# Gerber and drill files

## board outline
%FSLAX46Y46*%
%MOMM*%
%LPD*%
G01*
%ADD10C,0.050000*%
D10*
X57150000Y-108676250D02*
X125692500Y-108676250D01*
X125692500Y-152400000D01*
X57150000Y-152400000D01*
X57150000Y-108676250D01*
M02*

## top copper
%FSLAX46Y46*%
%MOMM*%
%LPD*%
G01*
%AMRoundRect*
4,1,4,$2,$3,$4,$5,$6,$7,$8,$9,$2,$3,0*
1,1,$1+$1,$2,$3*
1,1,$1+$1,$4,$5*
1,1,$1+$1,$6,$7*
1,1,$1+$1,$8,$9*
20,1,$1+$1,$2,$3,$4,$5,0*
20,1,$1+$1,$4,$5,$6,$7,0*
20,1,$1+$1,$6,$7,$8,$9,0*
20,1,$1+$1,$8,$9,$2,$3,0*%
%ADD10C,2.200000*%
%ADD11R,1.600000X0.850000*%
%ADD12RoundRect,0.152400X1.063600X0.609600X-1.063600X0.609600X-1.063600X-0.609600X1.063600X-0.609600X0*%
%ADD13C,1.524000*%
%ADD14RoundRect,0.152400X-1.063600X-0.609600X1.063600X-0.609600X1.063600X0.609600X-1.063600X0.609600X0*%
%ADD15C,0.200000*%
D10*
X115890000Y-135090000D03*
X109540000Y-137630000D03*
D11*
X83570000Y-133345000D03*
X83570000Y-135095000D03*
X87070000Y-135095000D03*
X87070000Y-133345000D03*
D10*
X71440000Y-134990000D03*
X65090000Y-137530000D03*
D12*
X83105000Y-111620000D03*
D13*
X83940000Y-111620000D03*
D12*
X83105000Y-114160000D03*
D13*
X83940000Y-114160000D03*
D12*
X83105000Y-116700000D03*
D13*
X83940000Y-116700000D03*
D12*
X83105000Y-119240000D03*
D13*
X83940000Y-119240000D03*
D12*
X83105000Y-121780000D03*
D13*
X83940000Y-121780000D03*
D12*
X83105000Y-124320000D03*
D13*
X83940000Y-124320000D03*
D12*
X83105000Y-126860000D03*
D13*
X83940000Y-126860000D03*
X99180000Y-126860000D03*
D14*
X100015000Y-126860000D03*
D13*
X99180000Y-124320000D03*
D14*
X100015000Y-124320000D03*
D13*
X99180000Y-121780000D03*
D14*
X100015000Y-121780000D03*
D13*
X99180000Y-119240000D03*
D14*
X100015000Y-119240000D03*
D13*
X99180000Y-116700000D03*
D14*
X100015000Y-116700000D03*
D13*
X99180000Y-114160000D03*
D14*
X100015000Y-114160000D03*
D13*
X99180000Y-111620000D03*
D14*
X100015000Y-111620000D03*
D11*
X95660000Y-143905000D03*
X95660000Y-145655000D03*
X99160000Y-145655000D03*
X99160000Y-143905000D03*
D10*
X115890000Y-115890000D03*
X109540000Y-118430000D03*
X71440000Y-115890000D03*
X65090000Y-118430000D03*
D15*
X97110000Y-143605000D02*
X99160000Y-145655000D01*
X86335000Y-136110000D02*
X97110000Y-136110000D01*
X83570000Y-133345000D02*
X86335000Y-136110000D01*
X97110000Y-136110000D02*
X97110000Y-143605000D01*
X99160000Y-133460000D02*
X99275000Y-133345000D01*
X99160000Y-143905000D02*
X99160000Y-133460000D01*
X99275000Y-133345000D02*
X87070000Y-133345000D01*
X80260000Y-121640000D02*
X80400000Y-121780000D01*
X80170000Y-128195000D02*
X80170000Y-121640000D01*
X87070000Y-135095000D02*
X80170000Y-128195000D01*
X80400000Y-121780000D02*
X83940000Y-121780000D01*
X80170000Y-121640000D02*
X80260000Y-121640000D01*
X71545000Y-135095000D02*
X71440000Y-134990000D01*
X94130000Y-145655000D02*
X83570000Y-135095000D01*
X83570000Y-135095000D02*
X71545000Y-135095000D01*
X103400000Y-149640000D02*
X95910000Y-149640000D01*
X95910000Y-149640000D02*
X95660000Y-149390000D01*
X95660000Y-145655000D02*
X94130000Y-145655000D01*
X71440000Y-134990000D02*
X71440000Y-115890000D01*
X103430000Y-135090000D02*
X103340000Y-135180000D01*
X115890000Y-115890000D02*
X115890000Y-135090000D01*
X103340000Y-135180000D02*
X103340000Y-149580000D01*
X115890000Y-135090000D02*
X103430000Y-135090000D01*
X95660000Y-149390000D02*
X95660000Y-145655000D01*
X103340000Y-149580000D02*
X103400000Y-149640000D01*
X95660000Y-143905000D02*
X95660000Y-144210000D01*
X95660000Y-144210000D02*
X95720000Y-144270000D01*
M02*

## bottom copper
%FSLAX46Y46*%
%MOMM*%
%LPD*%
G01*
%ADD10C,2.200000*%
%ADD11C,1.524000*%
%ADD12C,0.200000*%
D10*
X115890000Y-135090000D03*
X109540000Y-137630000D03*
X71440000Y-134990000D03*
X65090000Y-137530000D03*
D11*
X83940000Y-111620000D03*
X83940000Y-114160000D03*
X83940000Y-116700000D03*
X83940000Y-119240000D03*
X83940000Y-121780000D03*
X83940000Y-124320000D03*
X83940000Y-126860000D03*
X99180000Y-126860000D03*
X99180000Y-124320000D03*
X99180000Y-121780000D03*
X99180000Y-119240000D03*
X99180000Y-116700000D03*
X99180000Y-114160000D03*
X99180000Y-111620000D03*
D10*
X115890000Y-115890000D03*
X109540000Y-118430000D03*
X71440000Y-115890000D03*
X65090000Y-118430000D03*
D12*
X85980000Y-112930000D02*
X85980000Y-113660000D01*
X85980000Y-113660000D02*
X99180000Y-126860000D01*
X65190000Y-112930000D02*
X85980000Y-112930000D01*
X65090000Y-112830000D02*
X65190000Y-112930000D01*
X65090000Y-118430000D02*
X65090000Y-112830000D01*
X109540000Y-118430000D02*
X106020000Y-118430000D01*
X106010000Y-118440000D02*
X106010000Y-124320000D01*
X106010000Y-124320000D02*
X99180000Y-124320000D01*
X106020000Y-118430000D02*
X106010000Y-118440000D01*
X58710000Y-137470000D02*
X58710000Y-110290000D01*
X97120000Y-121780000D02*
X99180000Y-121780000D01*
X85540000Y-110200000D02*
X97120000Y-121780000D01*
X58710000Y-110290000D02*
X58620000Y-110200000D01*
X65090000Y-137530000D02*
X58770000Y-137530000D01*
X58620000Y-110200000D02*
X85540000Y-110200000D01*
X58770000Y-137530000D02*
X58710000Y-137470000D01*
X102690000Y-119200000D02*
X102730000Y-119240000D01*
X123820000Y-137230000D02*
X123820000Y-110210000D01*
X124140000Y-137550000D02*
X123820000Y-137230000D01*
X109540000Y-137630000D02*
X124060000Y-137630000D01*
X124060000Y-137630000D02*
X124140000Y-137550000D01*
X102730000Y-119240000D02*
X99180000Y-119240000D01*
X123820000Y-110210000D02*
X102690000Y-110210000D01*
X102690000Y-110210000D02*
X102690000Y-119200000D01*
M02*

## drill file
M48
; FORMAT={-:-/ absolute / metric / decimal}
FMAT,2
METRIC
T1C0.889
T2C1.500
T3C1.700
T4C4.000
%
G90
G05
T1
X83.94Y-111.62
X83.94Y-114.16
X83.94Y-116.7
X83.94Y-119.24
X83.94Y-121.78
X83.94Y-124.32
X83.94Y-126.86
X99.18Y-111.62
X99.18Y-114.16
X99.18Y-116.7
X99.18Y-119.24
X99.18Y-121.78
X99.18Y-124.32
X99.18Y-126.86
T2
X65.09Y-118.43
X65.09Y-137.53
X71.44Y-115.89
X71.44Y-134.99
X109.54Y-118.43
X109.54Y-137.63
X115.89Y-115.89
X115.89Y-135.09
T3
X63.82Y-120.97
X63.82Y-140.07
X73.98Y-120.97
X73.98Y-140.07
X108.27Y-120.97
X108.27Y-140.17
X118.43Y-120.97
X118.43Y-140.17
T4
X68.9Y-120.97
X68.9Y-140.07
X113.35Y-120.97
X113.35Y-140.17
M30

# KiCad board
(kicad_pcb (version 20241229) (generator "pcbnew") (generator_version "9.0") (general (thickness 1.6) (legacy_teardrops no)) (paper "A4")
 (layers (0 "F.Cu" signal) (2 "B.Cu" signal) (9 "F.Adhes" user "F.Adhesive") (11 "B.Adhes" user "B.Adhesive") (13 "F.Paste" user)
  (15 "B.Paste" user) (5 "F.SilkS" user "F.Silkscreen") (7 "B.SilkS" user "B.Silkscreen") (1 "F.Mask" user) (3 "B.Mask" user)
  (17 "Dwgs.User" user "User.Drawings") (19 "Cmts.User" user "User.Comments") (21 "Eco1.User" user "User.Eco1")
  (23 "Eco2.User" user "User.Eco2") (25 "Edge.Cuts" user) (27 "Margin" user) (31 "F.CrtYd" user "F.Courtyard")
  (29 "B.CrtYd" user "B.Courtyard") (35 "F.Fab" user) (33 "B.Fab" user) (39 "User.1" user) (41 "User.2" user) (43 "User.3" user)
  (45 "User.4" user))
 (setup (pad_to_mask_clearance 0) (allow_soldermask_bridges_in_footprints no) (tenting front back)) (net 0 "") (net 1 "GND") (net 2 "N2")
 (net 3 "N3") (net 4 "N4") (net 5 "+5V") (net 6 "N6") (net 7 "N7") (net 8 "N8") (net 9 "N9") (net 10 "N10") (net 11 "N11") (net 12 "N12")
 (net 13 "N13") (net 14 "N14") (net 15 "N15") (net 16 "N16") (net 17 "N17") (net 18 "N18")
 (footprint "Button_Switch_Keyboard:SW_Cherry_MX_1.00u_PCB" (layer "F.Cu") (at 115.89 135.09)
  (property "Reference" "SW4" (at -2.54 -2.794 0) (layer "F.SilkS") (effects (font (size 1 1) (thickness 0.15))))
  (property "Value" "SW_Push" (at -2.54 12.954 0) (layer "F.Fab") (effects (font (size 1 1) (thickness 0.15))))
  (pad "" np_thru_hole circle (at -7.62 5.08) (size 1.7 1.7) (drill 1.7) (layers "*.Cu" "*.Mask"))
  (pad "" np_thru_hole circle (at -2.54 5.08) (size 4 4) (drill 4) (layers "*.Cu" "*.Mask"))
  (pad "" np_thru_hole circle (at 2.54 5.08) (size 1.7 1.7) (drill 1.7) (layers "*.Cu" "*.Mask"))
  (pad "1" thru_hole circle (at 0 0) (size 2.2 2.2) (drill 1.5) (layers "*.Cu" "*.Mask") (remove_unused_layers no) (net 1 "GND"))
  (pad "2" thru_hole circle (at -6.35 2.54) (size 2.2 2.2) (drill 1.5) (layers "*.Cu" "*.Mask") (remove_unused_layers no) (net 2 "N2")))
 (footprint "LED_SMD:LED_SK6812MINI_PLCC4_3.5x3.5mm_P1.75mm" (layer "F.Cu") (at 85.32 134.22)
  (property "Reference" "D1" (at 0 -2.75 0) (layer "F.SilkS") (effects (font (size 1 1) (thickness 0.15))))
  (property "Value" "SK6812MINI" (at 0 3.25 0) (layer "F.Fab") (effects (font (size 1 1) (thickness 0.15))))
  (pad "1" smd rect (at -1.75 -0.875) (size 1.6 0.85) (layers "F.Cu" "F.Mask" "F.Paste") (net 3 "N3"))
  (pad "2" smd rect (at -1.75 0.875) (size 1.6 0.85) (layers "F.Cu" "F.Mask" "F.Paste") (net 1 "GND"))
  (pad "3" smd rect (at 1.75 0.875) (size 1.6 0.85) (layers "F.Cu" "F.Mask" "F.Paste") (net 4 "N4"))
  (pad "4" smd rect (at 1.75 -0.875) (size 1.6 0.85) (layers "F.Cu" "F.Mask" "F.Paste") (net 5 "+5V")))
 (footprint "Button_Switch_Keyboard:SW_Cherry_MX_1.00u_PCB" (layer "F.Cu") (at 71.44 134.99)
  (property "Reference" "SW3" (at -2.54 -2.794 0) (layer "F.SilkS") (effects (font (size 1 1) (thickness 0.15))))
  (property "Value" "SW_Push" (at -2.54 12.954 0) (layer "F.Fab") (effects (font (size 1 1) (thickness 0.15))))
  (pad "" np_thru_hole circle (at -7.62 5.08) (size 1.7 1.7) (drill 1.7) (layers "*.Cu" "*.Mask"))
  (pad "" np_thru_hole circle (at -2.54 5.08) (size 4 4) (drill 4) (layers "*.Cu" "*.Mask"))
  (pad "" np_thru_hole circle (at 2.54 5.08) (size 1.7 1.7) (drill 1.7) (layers "*.Cu" "*.Mask"))
  (pad "1" thru_hole circle (at 0 0) (size 2.2 2.2) (drill 1.5) (layers "*.Cu" "*.Mask") (remove_unused_layers no) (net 1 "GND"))
  (pad "2" thru_hole circle (at -6.35 2.54) (size 2.2 2.2) (drill 1.5) (layers "*.Cu" "*.Mask") (remove_unused_layers no) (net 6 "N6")))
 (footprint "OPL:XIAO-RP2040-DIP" (layer "F.Cu") (at 91.56 119.24)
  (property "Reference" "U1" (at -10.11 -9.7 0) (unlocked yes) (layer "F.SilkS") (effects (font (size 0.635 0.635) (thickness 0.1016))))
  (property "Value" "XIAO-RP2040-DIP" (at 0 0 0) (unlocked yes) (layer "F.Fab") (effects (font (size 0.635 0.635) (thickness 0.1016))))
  (pad "1" smd roundrect (at -8.455 -7.62 180) (size 2.432 1.524) (layers "F.Cu" "F.Mask") (roundrect_rratio 0.1) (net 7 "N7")
   (thermal_bridge_angle 45))
  (pad "1" thru_hole circle (at -7.62 -7.62 180) (size 1.524 1.524) (drill 0.889) (layers "*.Cu" "*.Mask") (remove_unused_layers no)
   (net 7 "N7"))
  (pad "2" smd roundrect (at -8.455 -5.08 180) (size 2.432 1.524) (layers "F.Cu" "F.Mask") (roundrect_rratio 0.1) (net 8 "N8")
   (thermal_bridge_angle 45))
  (pad "2" thru_hole circle (at -7.62 -5.08 180) (size 1.524 1.524) (drill 0.889) (layers "*.Cu" "*.Mask") (remove_unused_layers no)
   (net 8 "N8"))
  (pad "3" smd roundrect (at -8.455 -2.54 180) (size 2.432 1.524) (layers "F.Cu" "F.Mask") (roundrect_rratio 0.1) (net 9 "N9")
   (thermal_bridge_angle 45))
  (pad "3" thru_hole circle (at -7.62 -2.54 180) (size 1.524 1.524) (drill 0.889) (layers "*.Cu" "*.Mask") (remove_unused_layers no)
   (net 9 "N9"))
  (pad "4" smd roundrect (at -8.455 0 180) (size 2.432 1.524) (layers "F.Cu" "F.Mask") (roundrect_rratio 0.1) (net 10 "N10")
   (thermal_bridge_angle 45))
  (pad "4" thru_hole circle (at -7.62 0 180) (size 1.524 1.524) (drill 0.889) (layers "*.Cu" "*.Mask") (remove_unused_layers no)
   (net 10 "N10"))
  (pad "5" smd roundrect (at -8.455 2.54 180) (size 2.432 1.524) (layers "F.Cu" "F.Mask") (roundrect_rratio 0.1) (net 4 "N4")
   (thermal_bridge_angle 45))
  (pad "5" thru_hole circle (at -7.62 2.54 180) (size 1.524 1.524) (drill 0.889) (layers "*.Cu" "*.Mask") (remove_unused_layers no)
   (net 4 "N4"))
  (pad "6" smd roundrect (at -8.455 5.08 180) (size 2.432 1.524) (layers "F.Cu" "F.Mask") (roundrect_rratio 0.1) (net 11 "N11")
   (thermal_bridge_angle 45))
  (pad "6" thru_hole circle (at -7.62 5.08 180) (size 1.524 1.524) (drill 0.889) (layers "*.Cu" "*.Mask") (remove_unused_layers no)
   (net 11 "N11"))
  (pad "7" smd roundrect (at -8.455 7.62 180) (size 2.432 1.524) (layers "F.Cu" "F.Mask") (roundrect_rratio 0.1) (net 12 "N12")
   (thermal_bridge_angle 45))
  (pad "7" thru_hole circle (at -7.62 7.62 180) (size 1.524 1.524) (drill 0.889) (layers "*.Cu" "*.Mask") (remove_unused_layers no)
   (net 12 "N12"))
  (pad "8" thru_hole circle (at 7.62 7.62) (size 1.524 1.524) (drill 0.889) (layers "*.Cu" "*.Mask") (remove_unused_layers no)
   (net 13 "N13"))
  (pad "8" smd roundrect (at 8.455 7.62) (size 2.432 1.524) (layers "F.Cu" "F.Mask") (roundrect_rratio 0.1) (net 13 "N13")
   (thermal_bridge_angle 45))
  (pad "9" thru_hole circle (at 7.62 5.08) (size 1.524 1.524) (drill 0.889) (layers "*.Cu" "*.Mask") (remove_unused_layers no)
   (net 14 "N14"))
  (pad "9" smd roundrect (at 8.455 5.08) (size 2.432 1.524) (layers "F.Cu" "F.Mask") (roundrect_rratio 0.1) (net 14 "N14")
   (thermal_bridge_angle 45))
  (pad "10" thru_hole circle (at 7.62 2.54) (size 1.524 1.524) (drill 0.889) (layers "*.Cu" "*.Mask") (remove_unused_layers no) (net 6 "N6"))
  (pad "10" smd roundrect (at 8.455 2.54) (size 2.432 1.524) (layers "F.Cu" "F.Mask") (roundrect_rratio 0.1) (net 6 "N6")
   (thermal_bridge_angle 45))
  (pad "11" thru_hole circle (at 7.62 0) (size 1.524 1.524) (drill 0.889) (layers "*.Cu" "*.Mask") (remove_unused_layers no) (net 2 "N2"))
  (pad "11" smd roundrect (at 8.455 0) (size 2.432 1.524) (layers "F.Cu" "F.Mask") (roundrect_rratio 0.1) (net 2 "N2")
   (thermal_bridge_angle 45))
  (pad "12" thru_hole circle (at 7.62 -2.54) (size 1.524 1.524) (drill 0.889) (layers "*.Cu" "*.Mask") (remove_unused_layers no)
   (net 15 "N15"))
  (pad "12" smd roundrect (at 8.455 -2.54) (size 2.432 1.524) (layers "F.Cu" "F.Mask") (roundrect_rratio 0.1) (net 15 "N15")
   (thermal_bridge_angle 45))
  (pad "13" thru_hole circle (at 7.62 -5.08) (size 1.524 1.524) (drill 0.889) (layers "*.Cu" "*.Mask") (remove_unused_layers no)
   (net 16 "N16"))
  (pad "13" smd roundrect (at 8.455 -5.08) (size 2.432 1.524) (layers "F.Cu" "F.Mask") (roundrect_rratio 0.1) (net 16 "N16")
   (thermal_bridge_angle 45))
  (pad "14" thru_hole circle (at 7.62 -7.62) (size 1.524 1.524) (drill 0.889) (layers "*.Cu" "*.Mask") (remove_unused_layers no)
   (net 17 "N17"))
  (pad "14" smd roundrect (at 8.455 -7.62) (size 2.432 1.524) (layers "F.Cu" "F.Mask") (roundrect_rratio 0.1) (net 17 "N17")
   (thermal_bridge_angle 45)))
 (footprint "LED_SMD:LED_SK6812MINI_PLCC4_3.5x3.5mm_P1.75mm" (layer "F.Cu") (at 97.41 144.78)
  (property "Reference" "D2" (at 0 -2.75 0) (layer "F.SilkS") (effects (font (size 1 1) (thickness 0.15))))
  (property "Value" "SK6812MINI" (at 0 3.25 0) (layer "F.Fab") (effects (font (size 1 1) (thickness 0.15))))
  (pad "1" smd rect (at -1.75 -0.875) (size 1.6 0.85) (layers "F.Cu" "F.Mask" "F.Paste") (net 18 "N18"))
  (pad "2" smd rect (at -1.75 0.875) (size 1.6 0.85) (layers "F.Cu" "F.Mask" "F.Paste") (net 1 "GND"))
  (pad "3" smd rect (at 1.75 0.875) (size 1.6 0.85) (layers "F.Cu" "F.Mask" "F.Paste") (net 3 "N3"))
  (pad "4" smd rect (at 1.75 -0.875) (size 1.6 0.85) (layers "F.Cu" "F.Mask" "F.Paste") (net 5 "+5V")))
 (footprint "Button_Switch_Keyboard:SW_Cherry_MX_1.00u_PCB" (layer "F.Cu") (at 115.89 115.89)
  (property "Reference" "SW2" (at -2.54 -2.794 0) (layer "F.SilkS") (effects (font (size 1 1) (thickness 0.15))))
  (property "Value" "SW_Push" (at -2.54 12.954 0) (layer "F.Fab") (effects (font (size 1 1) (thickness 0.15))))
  (pad "" np_thru_hole circle (at -7.62 5.08) (size 1.7 1.7) (drill 1.7) (layers "*.Cu" "*.Mask"))
  (pad "" np_thru_hole circle (at -2.54 5.08) (size 4 4) (drill 4) (layers "*.Cu" "*.Mask"))
  (pad "" np_thru_hole circle (at 2.54 5.08) (size 1.7 1.7) (drill 1.7) (layers "*.Cu" "*.Mask"))
  (pad "1" thru_hole circle (at 0 0) (size 2.2 2.2) (drill 1.5) (layers "*.Cu" "*.Mask") (remove_unused_layers no) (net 1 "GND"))
  (pad "2" thru_hole circle (at -6.35 2.54) (size 2.2 2.2) (drill 1.5) (layers "*.Cu" "*.Mask") (remove_unused_layers no) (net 14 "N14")))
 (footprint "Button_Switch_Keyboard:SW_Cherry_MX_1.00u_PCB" (layer "F.Cu") (at 71.44 115.89)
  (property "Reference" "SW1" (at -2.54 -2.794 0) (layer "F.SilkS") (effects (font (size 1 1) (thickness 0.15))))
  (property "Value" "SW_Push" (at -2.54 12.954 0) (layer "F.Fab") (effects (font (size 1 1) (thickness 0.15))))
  (pad "" np_thru_hole circle (at -7.62 5.08) (size 1.7 1.7) (drill 1.7) (layers "*.Cu" "*.Mask"))
  (pad "" np_thru_hole circle (at -2.54 5.08) (size 4 4) (drill 4) (layers "*.Cu" "*.Mask"))
  (pad "" np_thru_hole circle (at 2.54 5.08) (size 1.7 1.7) (drill 1.7) (layers "*.Cu" "*.Mask"))
  (pad "1" thru_hole circle (at 0 0) (size 2.2 2.2) (drill 1.5) (layers "*.Cu" "*.Mask") (remove_unused_layers no) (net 1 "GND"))
  (pad "2" thru_hole circle (at -6.35 2.54) (size 2.2 2.2) (drill 1.5) (layers "*.Cu" "*.Mask") (remove_unused_layers no) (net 13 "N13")))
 (gr_rect (start 57.15 108.67625) (end 125.6925 152.4) (stroke (width 0.05) (type default)) (fill no) (layer "Edge.Cuts"))
 (segment (start 97.11 143.605) (end 99.16 145.655) (width 0.2) (layer "F.Cu") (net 3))
 (segment (start 86.335 136.11) (end 97.11 136.11) (width 0.2) (layer "F.Cu") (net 3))
 (segment (start 83.57 133.345) (end 86.335 136.11) (width 0.2) (layer "F.Cu") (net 3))
 (segment (start 97.11 136.11) (end 97.11 143.605) (width 0.2) (layer "F.Cu") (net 3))
 (segment (start 99.16 133.46) (end 99.275 133.345) (width 0.2) (layer "F.Cu") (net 5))
 (segment (start 99.16 143.905) (end 99.16 133.46) (width 0.2) (layer "F.Cu") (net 5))
 (segment (start 99.275 133.345) (end 87.07 133.345) (width 0.2) (layer "F.Cu") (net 5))
 (segment (start 80.26 121.64) (end 80.4 121.78) (width 0.2) (layer "F.Cu") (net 4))
 (segment (start 80.17 128.195) (end 80.17 121.64) (width 0.2) (layer "F.Cu") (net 4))
 (segment (start 87.07 135.095) (end 80.17 128.195) (width 0.2) (layer "F.Cu") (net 4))
 (segment (start 80.4 121.78) (end 83.94 121.78) (width 0.2) (layer "F.Cu") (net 4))
 (segment (start 80.17 121.64) (end 80.26 121.64) (width 0.2) (layer "F.Cu") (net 4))
 (segment (start 71.545 135.095) (end 71.44 134.99) (width 0.2) (layer "F.Cu") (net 1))
 (segment (start 94.13 145.655) (end 83.57 135.095) (width 0.2) (layer "F.Cu") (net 1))
 (segment (start 83.57 135.095) (end 71.545 135.095) (width 0.2) (layer "F.Cu") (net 1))
 (segment (start 103.4 149.64) (end 95.91 149.64) (width 0.2) (layer "F.Cu") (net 1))
 (segment (start 95.91 149.64) (end 95.66 149.39) (width 0.2) (layer "F.Cu") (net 1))
 (segment (start 95.66 145.655) (end 94.13 145.655) (width 0.2) (layer "F.Cu") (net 1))
 (segment (start 71.44 134.99) (end 71.44 115.89) (width 0.2) (layer "F.Cu") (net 1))
 (segment (start 103.43 135.09) (end 103.34 135.18) (width 0.2) (layer "F.Cu") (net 1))
 (segment (start 115.89 115.89) (end 115.89 135.09) (width 0.2) (layer "F.Cu") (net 1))
 (segment (start 103.34 135.18) (end 103.34 149.58) (width 0.2) (layer "F.Cu") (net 1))
 (segment (start 115.89 135.09) (end 103.43 135.09) (width 0.2) (layer "F.Cu") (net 1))
 (segment (start 95.66 149.39) (end 95.66 145.655) (width 0.2) (layer "F.Cu") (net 1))
 (segment (start 103.34 149.58) (end 103.4 149.64) (width 0.2) (layer "F.Cu") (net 1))
 (segment (start 95.66 143.905) (end 95.66 144.21) (width 0.2) (layer "F.Cu") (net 18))
 (segment (start 95.66 144.21) (end 95.72 144.27) (width 0.2) (layer "F.Cu") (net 18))
 (segment (start 85.98 112.93) (end 85.98 113.66) (width 0.2) (layer "B.Cu") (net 13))
 (segment (start 85.98 113.66) (end 99.18 126.86) (width 0.2) (layer "B.Cu") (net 13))
 (segment (start 65.19 112.93) (end 85.98 112.93) (width 0.2) (layer "B.Cu") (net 13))
 (segment (start 65.09 112.83) (end 65.19 112.93) (width 0.2) (layer "B.Cu") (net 13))
 (segment (start 65.09 118.43) (end 65.09 112.83) (width 0.2) (layer "B.Cu") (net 13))
 (segment (start 109.54 118.43) (end 106.02 118.43) (width 0.2) (layer "B.Cu") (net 14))
 (segment (start 106.01 118.44) (end 106.01 124.32) (width 0.2) (layer "B.Cu") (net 14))
 (segment (start 106.01 124.32) (end 99.18 124.32) (width 0.2) (layer "B.Cu") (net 14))
 (segment (start 106.02 118.43) (end 106.01 118.44) (width 0.2) (layer "B.Cu") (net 14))
 (segment (start 58.71 137.47) (end 58.71 110.29) (width 0.2) (layer "B.Cu") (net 6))
 (segment (start 97.12 121.78) (end 99.18 121.78) (width 0.2) (layer "B.Cu") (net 6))
 (segment (start 85.54 110.2) (end 97.12 121.78) (width 0.2) (layer "B.Cu") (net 6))
 (segment (start 58.71 110.29) (end 58.62 110.2) (width 0.2) (layer "B.Cu") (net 6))
 (segment (start 65.09 137.53) (end 58.77 137.53) (width 0.2) (layer "B.Cu") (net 6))
 (segment (start 58.62 110.2) (end 85.54 110.2) (width 0.2) (layer "B.Cu") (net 6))
 (segment (start 58.77 137.53) (end 58.71 137.47) (width 0.2) (layer "B.Cu") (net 6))
 (segment (start 102.69 119.2) (end 102.73 119.24) (width 0.2) (layer "B.Cu") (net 2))
 (segment (start 123.82 137.23) (end 123.82 110.21) (width 0.2) (layer "B.Cu") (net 2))
 (segment (start 124.14 137.55) (end 123.82 137.23) (width 0.2) (layer "B.Cu") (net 2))
 (segment (start 109.54 137.63) (end 124.06 137.63) (width 0.2) (layer "B.Cu") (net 2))
 (segment (start 124.06 137.63) (end 124.14 137.55) (width 0.2) (layer "B.Cu") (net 2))
 (segment (start 102.73 119.24) (end 99.18 119.24) (width 0.2) (layer "B.Cu") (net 2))
 (segment (start 123.82 110.21) (end 102.69 110.21) (width 0.2) (layer "B.Cu") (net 2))
 (segment (start 102.69 110.21) (end 102.69 119.2) (width 0.2) (layer "B.Cu") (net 2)))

